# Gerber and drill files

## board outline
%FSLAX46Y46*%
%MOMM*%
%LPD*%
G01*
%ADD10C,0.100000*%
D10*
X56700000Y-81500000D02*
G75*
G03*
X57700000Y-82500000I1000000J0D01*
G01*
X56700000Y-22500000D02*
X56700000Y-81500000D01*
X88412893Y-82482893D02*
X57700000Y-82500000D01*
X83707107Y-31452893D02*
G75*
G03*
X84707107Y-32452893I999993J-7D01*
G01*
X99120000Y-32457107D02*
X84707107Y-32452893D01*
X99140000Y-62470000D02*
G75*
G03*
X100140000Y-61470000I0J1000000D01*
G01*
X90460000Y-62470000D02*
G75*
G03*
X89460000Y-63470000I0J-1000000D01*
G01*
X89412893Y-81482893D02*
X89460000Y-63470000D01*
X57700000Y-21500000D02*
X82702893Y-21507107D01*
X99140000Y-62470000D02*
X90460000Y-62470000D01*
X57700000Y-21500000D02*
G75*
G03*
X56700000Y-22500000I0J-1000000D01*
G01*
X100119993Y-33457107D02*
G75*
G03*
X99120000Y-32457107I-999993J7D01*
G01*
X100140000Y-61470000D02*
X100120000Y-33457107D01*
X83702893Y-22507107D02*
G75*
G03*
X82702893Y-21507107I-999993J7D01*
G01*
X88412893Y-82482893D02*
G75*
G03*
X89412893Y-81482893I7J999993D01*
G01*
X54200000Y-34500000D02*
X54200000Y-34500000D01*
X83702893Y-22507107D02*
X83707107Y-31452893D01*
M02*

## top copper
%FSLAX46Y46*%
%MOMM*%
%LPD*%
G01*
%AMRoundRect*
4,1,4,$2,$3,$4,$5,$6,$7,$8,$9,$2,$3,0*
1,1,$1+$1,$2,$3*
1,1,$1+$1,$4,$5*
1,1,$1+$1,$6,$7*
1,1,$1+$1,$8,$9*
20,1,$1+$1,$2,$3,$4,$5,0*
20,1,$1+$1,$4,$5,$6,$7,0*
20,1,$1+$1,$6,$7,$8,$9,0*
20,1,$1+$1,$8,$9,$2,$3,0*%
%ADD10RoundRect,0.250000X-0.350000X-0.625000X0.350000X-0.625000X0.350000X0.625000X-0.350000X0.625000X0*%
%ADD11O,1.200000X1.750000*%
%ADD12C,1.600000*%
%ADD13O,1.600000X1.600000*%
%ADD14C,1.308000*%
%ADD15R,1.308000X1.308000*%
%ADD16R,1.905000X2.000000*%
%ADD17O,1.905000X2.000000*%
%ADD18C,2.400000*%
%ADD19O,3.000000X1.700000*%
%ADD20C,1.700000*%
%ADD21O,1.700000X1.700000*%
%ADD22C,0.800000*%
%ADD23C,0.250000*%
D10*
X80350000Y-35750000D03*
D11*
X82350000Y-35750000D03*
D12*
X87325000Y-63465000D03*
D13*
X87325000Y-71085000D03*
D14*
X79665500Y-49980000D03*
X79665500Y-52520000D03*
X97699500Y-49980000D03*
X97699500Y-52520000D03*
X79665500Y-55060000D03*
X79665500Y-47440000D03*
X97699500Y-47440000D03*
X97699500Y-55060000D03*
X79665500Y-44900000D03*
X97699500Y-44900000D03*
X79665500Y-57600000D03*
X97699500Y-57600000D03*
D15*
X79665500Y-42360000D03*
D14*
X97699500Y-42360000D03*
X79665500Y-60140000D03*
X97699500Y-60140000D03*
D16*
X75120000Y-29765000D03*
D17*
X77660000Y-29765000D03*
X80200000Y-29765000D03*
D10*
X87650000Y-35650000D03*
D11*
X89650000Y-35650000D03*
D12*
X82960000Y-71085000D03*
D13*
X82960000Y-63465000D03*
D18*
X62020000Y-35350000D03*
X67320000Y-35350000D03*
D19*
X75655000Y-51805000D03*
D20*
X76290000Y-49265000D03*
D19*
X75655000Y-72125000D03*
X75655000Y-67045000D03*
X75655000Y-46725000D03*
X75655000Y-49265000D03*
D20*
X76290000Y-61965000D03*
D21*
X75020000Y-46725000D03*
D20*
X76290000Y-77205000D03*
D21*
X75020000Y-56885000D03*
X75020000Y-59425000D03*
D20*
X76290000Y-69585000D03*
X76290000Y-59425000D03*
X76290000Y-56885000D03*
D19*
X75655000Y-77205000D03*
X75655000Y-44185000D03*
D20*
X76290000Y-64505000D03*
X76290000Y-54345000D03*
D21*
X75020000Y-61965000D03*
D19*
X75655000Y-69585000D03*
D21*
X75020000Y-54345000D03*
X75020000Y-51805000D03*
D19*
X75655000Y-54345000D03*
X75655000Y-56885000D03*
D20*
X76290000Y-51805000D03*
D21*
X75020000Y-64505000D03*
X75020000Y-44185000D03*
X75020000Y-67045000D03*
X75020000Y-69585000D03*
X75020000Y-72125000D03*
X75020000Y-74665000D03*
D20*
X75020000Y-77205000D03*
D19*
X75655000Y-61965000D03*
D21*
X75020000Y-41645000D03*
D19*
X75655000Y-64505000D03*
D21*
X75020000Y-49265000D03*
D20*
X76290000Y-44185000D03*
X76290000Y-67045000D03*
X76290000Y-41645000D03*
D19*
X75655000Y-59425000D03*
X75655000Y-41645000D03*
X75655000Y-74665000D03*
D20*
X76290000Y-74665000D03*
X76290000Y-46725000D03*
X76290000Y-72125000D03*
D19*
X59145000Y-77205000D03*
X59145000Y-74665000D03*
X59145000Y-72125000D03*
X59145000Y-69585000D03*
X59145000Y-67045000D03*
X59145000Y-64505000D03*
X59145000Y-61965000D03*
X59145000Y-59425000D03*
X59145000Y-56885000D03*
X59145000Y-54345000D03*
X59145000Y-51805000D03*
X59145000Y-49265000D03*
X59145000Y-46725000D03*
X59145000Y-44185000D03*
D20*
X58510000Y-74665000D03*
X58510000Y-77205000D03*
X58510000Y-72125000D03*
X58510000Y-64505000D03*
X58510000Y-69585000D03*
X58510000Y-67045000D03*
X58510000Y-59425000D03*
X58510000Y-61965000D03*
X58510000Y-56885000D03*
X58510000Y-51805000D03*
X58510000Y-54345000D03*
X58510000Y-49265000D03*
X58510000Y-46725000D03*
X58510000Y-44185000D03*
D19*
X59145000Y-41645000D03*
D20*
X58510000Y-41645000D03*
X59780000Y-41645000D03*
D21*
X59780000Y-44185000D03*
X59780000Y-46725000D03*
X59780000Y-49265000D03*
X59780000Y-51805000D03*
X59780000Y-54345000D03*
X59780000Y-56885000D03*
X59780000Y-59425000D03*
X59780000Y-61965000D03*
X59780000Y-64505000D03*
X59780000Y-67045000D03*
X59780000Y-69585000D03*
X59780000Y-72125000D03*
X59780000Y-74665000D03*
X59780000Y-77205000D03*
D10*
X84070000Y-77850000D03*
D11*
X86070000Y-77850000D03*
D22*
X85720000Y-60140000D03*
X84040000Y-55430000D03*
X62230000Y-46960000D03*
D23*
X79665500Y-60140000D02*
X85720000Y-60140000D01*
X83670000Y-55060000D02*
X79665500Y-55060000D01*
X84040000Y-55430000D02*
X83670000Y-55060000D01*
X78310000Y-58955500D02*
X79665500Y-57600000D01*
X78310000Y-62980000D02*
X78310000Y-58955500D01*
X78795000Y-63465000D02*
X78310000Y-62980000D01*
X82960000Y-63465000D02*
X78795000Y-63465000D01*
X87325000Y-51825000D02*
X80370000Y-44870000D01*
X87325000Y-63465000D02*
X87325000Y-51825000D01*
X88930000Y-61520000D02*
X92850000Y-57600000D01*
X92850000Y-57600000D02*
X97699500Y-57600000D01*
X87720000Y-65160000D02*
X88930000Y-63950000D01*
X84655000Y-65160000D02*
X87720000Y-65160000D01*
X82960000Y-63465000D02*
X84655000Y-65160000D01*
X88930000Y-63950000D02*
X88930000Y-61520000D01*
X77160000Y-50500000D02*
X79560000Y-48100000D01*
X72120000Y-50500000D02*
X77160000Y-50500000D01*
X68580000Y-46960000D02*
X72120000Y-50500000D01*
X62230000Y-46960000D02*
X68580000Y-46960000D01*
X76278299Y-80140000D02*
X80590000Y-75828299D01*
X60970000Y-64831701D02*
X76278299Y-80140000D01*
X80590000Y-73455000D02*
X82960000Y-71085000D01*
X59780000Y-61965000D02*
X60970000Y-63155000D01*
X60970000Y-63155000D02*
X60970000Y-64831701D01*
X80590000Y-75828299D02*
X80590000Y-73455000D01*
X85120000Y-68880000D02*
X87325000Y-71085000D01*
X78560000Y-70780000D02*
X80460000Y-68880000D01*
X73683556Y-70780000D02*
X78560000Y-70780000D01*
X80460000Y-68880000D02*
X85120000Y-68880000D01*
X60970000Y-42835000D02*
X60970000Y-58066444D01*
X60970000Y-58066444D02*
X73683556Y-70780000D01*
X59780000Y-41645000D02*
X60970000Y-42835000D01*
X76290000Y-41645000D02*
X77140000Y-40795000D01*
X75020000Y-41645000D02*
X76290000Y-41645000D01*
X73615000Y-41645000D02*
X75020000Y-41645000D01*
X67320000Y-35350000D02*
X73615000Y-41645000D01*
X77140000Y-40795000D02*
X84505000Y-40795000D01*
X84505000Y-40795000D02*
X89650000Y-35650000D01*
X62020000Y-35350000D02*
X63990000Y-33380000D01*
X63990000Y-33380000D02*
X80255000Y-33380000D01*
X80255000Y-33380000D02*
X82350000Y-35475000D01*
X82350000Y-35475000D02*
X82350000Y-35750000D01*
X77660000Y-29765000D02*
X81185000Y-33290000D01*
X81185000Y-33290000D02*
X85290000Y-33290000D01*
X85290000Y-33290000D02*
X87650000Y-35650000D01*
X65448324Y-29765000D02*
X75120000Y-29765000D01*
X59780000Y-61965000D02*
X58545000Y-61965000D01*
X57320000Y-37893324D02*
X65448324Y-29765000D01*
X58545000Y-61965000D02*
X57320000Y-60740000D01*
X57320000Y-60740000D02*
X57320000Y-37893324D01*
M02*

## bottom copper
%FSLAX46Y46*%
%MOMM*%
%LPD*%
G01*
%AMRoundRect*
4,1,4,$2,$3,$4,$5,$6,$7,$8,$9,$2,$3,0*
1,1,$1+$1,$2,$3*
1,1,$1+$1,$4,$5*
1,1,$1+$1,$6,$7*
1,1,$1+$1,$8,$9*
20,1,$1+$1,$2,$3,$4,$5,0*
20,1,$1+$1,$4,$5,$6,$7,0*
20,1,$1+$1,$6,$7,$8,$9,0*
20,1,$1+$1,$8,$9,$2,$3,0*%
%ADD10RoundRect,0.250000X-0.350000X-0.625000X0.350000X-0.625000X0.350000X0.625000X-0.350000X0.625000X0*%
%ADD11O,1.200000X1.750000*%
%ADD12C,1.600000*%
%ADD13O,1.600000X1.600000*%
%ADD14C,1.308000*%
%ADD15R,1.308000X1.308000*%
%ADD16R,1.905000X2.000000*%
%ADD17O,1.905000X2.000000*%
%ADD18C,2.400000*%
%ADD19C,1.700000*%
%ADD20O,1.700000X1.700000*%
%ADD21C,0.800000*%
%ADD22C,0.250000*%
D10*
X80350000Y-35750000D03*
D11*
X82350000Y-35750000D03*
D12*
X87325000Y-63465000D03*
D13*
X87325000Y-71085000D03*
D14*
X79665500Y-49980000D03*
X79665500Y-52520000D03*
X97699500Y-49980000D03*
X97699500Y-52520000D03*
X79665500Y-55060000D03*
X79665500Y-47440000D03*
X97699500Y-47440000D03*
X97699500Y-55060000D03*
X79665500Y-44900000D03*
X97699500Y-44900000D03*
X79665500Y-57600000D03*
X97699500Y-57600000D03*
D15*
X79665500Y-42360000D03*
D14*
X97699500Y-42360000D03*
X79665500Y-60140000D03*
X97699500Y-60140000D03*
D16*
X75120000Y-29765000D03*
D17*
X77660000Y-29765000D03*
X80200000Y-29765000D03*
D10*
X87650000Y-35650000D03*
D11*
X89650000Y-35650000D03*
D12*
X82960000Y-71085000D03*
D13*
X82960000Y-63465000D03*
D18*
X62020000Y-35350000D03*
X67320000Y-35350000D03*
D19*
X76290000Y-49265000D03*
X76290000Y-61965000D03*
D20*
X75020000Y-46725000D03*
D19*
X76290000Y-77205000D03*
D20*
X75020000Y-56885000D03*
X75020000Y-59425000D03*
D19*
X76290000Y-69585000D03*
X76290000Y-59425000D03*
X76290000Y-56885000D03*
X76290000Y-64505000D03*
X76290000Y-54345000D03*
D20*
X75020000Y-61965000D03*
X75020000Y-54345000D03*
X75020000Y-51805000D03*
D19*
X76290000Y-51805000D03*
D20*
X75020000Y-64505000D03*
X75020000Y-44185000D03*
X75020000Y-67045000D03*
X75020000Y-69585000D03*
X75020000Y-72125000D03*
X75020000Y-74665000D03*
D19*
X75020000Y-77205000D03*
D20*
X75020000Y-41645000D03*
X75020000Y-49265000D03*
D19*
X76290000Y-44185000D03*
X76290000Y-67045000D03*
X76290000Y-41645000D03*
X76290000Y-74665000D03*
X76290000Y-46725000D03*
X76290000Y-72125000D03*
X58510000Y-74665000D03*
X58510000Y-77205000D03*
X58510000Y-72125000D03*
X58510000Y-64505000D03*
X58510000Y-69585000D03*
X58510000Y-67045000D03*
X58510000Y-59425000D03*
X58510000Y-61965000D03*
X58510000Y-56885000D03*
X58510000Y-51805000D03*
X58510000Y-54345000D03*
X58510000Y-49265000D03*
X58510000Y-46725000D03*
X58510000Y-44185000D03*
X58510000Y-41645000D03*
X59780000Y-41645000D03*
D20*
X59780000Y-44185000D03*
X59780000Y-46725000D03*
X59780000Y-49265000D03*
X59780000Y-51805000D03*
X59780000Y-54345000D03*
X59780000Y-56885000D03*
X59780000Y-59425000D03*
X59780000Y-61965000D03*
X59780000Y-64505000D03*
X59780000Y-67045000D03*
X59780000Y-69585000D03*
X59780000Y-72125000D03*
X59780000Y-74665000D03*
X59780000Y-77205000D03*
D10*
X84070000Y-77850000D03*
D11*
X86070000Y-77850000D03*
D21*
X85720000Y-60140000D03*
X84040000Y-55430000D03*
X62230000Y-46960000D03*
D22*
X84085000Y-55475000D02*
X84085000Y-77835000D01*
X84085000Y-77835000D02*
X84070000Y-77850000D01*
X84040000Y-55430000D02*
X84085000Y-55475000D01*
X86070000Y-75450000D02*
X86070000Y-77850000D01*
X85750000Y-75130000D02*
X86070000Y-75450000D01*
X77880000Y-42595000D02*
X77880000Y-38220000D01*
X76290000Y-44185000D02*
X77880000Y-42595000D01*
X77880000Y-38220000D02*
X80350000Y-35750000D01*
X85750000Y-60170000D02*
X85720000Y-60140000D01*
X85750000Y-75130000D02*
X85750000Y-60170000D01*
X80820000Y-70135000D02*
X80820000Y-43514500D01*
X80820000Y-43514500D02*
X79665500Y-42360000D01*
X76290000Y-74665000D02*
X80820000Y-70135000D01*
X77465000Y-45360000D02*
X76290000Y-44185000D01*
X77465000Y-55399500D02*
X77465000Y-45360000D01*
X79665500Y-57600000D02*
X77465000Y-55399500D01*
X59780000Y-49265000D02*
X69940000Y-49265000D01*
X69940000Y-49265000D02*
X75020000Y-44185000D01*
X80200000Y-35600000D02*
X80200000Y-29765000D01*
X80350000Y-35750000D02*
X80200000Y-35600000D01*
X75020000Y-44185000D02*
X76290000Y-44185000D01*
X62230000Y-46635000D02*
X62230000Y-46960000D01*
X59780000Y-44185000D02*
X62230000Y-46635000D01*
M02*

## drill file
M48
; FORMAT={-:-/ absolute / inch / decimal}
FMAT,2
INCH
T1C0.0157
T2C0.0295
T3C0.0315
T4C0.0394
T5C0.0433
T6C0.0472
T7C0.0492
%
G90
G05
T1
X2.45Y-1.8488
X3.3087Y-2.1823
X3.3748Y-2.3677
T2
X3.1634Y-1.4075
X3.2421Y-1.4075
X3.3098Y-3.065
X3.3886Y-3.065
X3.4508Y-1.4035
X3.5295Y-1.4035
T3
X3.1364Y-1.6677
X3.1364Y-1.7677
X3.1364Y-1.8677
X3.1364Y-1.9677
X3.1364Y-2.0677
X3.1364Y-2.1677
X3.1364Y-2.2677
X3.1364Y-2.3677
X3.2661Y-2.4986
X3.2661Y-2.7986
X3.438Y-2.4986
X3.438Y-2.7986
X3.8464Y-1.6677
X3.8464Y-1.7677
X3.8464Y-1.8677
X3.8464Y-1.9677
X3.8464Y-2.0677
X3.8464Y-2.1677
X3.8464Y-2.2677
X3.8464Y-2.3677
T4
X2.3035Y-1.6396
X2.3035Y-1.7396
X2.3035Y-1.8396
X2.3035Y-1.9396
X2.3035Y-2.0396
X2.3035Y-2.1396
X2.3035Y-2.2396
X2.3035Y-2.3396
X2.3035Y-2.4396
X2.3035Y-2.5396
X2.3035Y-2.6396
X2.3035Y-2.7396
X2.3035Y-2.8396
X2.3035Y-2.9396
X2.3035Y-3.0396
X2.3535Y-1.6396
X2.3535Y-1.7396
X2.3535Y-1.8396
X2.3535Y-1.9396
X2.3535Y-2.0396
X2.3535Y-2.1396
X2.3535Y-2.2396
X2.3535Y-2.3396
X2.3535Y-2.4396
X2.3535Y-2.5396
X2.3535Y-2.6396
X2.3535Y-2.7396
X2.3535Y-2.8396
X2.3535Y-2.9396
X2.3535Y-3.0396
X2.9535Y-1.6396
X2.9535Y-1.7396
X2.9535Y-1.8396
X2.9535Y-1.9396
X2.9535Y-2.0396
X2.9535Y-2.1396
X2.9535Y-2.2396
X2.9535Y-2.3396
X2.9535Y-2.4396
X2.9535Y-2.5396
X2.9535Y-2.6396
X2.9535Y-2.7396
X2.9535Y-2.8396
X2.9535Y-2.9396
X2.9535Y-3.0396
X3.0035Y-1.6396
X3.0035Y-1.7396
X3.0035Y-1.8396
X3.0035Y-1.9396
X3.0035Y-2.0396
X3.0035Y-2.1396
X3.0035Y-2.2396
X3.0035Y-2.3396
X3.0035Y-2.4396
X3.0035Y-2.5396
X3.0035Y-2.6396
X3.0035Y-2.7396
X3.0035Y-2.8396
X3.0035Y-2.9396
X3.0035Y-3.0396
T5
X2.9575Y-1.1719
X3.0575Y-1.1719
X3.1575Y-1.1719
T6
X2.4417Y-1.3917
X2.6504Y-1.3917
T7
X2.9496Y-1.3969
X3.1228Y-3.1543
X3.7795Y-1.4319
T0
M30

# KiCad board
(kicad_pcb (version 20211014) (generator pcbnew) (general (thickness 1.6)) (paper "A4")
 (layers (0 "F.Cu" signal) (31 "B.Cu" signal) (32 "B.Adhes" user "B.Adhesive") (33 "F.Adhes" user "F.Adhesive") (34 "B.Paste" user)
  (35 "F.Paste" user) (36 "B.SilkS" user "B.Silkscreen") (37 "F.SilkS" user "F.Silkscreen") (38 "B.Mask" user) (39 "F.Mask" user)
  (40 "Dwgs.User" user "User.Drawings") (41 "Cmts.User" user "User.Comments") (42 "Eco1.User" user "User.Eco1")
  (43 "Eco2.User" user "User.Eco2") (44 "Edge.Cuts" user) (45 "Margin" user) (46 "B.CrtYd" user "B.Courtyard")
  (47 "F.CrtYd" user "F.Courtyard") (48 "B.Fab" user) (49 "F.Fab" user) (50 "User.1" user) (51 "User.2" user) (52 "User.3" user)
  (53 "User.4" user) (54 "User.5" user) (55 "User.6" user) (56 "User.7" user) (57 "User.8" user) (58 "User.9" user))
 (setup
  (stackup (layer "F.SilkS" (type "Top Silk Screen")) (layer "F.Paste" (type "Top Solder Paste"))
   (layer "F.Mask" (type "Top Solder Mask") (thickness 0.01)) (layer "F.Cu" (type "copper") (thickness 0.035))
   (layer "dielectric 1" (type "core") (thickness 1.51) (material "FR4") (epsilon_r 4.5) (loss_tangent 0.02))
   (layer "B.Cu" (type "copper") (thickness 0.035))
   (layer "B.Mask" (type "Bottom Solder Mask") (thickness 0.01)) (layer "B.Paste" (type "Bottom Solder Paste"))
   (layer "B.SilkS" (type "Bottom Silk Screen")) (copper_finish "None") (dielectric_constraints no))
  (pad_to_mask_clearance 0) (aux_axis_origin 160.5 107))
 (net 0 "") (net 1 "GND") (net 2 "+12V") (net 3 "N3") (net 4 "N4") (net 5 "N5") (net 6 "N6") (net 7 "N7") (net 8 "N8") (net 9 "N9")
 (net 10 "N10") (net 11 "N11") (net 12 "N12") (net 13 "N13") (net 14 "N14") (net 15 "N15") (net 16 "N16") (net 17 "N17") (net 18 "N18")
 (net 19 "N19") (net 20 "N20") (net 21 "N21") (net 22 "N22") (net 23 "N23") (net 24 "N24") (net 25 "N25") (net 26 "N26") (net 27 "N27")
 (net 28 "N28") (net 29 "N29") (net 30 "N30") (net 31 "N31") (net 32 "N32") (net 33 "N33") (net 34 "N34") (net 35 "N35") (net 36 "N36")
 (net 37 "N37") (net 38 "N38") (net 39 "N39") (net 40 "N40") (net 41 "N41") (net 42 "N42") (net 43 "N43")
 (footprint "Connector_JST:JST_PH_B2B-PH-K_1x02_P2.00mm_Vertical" (layer "F.Cu") (at 80.35 35.75)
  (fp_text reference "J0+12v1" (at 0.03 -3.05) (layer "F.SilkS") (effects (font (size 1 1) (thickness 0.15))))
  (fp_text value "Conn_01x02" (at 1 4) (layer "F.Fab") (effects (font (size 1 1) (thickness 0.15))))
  (pad "1" thru_hole roundrect (at 0 0) (size 1.2 1.75) (drill 0.75) (layers *.Cu *.Mask) (roundrect_rratio 0.208333) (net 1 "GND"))
  (pad "2" thru_hole oval (at 2 0) (size 1.2 1.75) (drill 0.75) (layers *.Cu *.Mask) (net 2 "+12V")))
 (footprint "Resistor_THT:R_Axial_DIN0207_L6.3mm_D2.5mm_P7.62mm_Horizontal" (layer "F.Cu") (at 87.325 63.465 -90)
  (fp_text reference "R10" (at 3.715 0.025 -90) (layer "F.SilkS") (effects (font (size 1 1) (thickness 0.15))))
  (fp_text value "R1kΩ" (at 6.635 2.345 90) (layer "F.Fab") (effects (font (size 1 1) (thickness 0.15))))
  (pad "1" thru_hole circle (at 0 0 270) (size 1.6 1.6) (drill 0.8) (layers *.Cu *.Mask) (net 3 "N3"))
  (pad "2" thru_hole oval (at 7.62 0 270) (size 1.6 1.6) (drill 0.8) (layers *.Cu *.Mask) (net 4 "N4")))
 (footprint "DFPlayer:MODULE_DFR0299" (layer "F.Cu") (at 88.6825 51.25)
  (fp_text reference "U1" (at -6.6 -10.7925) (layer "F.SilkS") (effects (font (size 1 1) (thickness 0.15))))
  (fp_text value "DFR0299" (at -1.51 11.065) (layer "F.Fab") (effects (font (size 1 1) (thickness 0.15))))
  (pad "1" thru_hole rect locked (at -9.017 -8.89) (size 1.308 1.308) (drill 0.8) (layers *.Cu *.Mask) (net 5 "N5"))
  (pad "2" thru_hole circle locked (at -9.017 -6.35) (size 1.308 1.308) (drill 0.8) (layers *.Cu *.Mask) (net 3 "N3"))
  (pad "3" thru_hole circle locked (at -9.017 -3.81) (size 1.308 1.308) (drill 0.8) (layers *.Cu *.Mask) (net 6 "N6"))
  (pad "4" thru_hole circle locked (at -9.017 -1.27) (size 1.308 1.308) (drill 0.8) (layers *.Cu *.Mask) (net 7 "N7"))
  (pad "5" thru_hole circle locked (at -9.017 1.27) (size 1.308 1.308) (drill 0.8) (layers *.Cu *.Mask) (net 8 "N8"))
  (pad "6" thru_hole circle locked (at -9.017 3.81) (size 1.308 1.308) (drill 0.8) (layers *.Cu *.Mask) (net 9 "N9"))
  (pad "7" thru_hole circle locked (at -9.017 6.35) (size 1.308 1.308) (drill 0.8) (layers *.Cu *.Mask) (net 1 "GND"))
  (pad "8" thru_hole circle locked (at -9.017 8.89) (size 1.308 1.308) (drill 0.8) (layers *.Cu *.Mask) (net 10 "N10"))
  (pad "9" thru_hole circle locked (at 9.017 8.89) (size 1.308 1.308) (drill 0.8) (layers *.Cu *.Mask) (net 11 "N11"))
  (pad "10" thru_hole circle locked (at 9.017 6.35) (size 1.308 1.308) (drill 0.8) (layers *.Cu *.Mask) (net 1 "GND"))
  (pad "11" thru_hole circle locked (at 9.017 3.81) (size 1.308 1.308) (drill 0.8) (layers *.Cu *.Mask) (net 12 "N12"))
  (pad "12" thru_hole circle locked (at 9.017 1.27) (size 1.308 1.308) (drill 0.8) (layers *.Cu *.Mask) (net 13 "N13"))
  (pad "13" thru_hole circle locked (at 9.017 -1.27) (size 1.308 1.308) (drill 0.8) (layers *.Cu *.Mask) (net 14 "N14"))
  (pad "14" thru_hole circle locked (at 9.017 -3.81) (size 1.308 1.308) (drill 0.8) (layers *.Cu *.Mask) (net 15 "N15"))
  (pad "15" thru_hole circle locked (at 9.017 -6.35) (size 1.308 1.308) (drill 0.8) (layers *.Cu *.Mask) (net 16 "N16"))
  (pad "16" thru_hole circle locked (at 9.017 -8.89) (size 1.308 1.308) (drill 0.8) (layers *.Cu *.Mask) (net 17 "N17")))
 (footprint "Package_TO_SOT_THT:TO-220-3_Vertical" (layer "F.Cu") (at 75.12 29.765)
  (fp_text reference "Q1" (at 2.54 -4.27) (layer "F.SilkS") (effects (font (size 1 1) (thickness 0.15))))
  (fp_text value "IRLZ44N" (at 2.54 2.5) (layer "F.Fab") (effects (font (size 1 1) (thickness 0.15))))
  (pad "1" thru_hole rect (at 0 0) (size 1.905 2) (drill 1.1) (layers *.Cu *.Mask) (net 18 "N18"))
  (pad "2" thru_hole oval (at 2.54 0) (size 1.905 2) (drill 1.1) (layers *.Cu *.Mask) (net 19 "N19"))
  (pad "3" thru_hole oval (at 5.08 0) (size 1.905 2) (drill 1.1) (layers *.Cu *.Mask) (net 1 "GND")))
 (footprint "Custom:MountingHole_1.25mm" (layer "F.Cu") (at 96 36.37)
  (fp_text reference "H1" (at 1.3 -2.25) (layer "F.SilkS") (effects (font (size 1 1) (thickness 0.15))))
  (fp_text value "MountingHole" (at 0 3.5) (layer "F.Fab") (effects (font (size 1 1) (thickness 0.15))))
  (pad "" np_thru_hole circle (at 0 0) (size 1.25 1.25) (drill 1.25) (layers F&B.Cu *.Mask)))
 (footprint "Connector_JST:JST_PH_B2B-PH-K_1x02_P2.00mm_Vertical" (layer "F.Cu") (at 87.65 35.65)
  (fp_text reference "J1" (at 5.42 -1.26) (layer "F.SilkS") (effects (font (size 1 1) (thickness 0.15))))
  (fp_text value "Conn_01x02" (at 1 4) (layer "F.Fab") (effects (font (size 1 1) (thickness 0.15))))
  (pad "1" thru_hole roundrect (at 0 0) (size 1.2 1.75) (drill 0.75) (layers *.Cu *.Mask) (roundrect_rratio 0.208333) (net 19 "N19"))
  (pad "2" thru_hole oval (at 2 0) (size 1.2 1.75) (drill 0.75) (layers *.Cu *.Mask) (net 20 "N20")))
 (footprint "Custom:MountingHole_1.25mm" (layer "F.Cu") (at 79.32 80.12)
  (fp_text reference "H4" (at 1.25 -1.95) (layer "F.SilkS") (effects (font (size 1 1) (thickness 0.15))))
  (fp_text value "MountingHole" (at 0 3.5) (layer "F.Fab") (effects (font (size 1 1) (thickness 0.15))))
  (pad "" np_thru_hole circle (at 0 0) (size 1.25 1.25) (drill 1.25) (layers F&B.Cu *.Mask)))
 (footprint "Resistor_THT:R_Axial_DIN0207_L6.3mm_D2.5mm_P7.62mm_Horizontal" (layer "F.Cu") (at 82.96 71.085 90)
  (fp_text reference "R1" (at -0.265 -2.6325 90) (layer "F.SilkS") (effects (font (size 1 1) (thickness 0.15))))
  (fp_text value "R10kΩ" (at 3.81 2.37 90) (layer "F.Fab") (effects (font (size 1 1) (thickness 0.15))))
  (pad "1" thru_hole circle (at 0 0 90) (size 1.6 1.6) (drill 0.8) (layers *.Cu *.Mask) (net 18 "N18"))
  (pad "2" thru_hole oval (at 7.62 0 90) (size 1.6 1.6) (drill 0.8) (layers *.Cu *.Mask) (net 1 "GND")))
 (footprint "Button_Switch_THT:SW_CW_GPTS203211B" (layer "F.Cu") (at 62.02 35.35 90)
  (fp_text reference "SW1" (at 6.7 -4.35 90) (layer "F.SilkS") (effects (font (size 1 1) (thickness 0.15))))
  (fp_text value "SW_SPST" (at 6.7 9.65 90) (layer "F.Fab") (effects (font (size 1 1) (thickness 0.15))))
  (pad "1" thru_hole circle (at 0 0 90) (size 2.4 2.4) (drill 1.2) (layers *.Cu *.Mask) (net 2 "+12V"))
  (pad "2" thru_hole circle (at 0 5.3 90) (size 2.4 2.4) (drill 1.2) (layers *.Cu *.Mask) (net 20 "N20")))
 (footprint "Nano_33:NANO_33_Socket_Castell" (layer "F.Cu") (at 67.4 59.425 90)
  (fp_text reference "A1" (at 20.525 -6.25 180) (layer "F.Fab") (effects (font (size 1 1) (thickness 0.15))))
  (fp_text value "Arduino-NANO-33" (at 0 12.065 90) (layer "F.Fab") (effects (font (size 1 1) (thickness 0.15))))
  (pad "1" thru_hole circle locked (at -17.78 7.62 180) (size 1.7 1.7) (drill 1) (layers *.Cu *.Mask) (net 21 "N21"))
  (pad "1" smd oval locked (at -17.78 8.255 180) (size 3 1.7) (layers "F.Cu" "F.Mask") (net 21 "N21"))
  (pad "1" thru_hole circle locked (at -17.78 8.89 180) (size 1.7 1.7) (drill 1) (layers *.Cu *.Mask) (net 21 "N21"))
  (pad "2" thru_hole oval locked (at -15.24 7.62 180) (size 1.7 1.7) (drill 1) (layers *.Cu *.Mask) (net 5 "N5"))
  (pad "2" smd oval locked (at -15.24 8.255 180) (size 3 1.7) (layers "F.Cu" "F.Mask") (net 5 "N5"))
  (pad "2" thru_hole circle locked (at -15.24 8.89 180) (size 1.7 1.7) (drill 1) (layers *.Cu *.Mask) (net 5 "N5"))
  (pad "3" smd oval locked (at -12.7 8.255 180) (size 3 1.7) (layers "F.Cu" "F.Mask") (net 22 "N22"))
  (pad "3" thru_hole oval locked (at -12.7 7.62 180) (size 1.7 1.7) (drill 1) (layers *.Cu *.Mask) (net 22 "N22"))
  (pad "3" thru_hole circle locked (at -12.7 8.89 180) (size 1.7 1.7) (drill 1) (layers *.Cu *.Mask) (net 22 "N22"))
  (pad "4" thru_hole circle locked (at -10.16 8.89 180) (size 1.7 1.7) (drill 1) (layers *.Cu *.Mask) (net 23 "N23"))
  (pad "4" smd oval locked (at -10.16 8.255 180) (size 3 1.7) (layers "F.Cu" "F.Mask") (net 23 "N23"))
  (pad "4" thru_hole oval locked (at -10.16 7.62 180) (size 1.7 1.7) (drill 1) (layers *.Cu *.Mask) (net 23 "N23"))
  (pad "5" thru_hole circle locked (at -7.62 8.89 180) (size 1.7 1.7) (drill 1) (layers *.Cu *.Mask) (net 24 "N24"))
  (pad "5" thru_hole oval locked (at -7.62 7.62 180) (size 1.7 1.7) (drill 1) (layers *.Cu *.Mask) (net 24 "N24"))
  (pad "5" smd oval locked (at -7.62 8.255 180) (size 3 1.7) (layers "F.Cu" "F.Mask") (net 24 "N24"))
  (pad "6" smd oval locked (at -5.08 8.255 180) (size 3 1.7) (layers "F.Cu" "F.Mask") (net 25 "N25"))
  (pad "6" thru_hole circle locked (at -5.08 8.89 180) (size 1.7 1.7) (drill 1) (layers *.Cu *.Mask) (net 25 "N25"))
  (pad "6" thru_hole oval locked (at -5.08 7.62 180) (size 1.7 1.7) (drill 1) (layers *.Cu *.Mask) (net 25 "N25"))
  (pad "7" thru_hole circle locked (at -2.54 8.89 180) (size 1.7 1.7) (drill 1) (layers *.Cu *.Mask) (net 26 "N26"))
  (pad "7" thru_hole oval locked (at -2.54 7.62 180) (size 1.7 1.7) (drill 1) (layers *.Cu *.Mask) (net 26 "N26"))
  (pad "7" smd oval locked (at -2.54 8.255 180) (size 3 1.7) (layers "F.Cu" "F.Mask") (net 26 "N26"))
  (pad "8" thru_hole oval locked (at 0 7.62 180) (size 1.7 1.7) (drill 1) (layers *.Cu *.Mask) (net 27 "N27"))
  (pad "8" smd oval locked (at 0 8.255 180) (size 3 1.7) (layers "F.Cu" "F.Mask") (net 27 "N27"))
  (pad "8" thru_hole circle locked (at 0 8.89 180) (size 1.7 1.7) (drill 1) (layers *.Cu *.Mask) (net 27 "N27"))
  (pad "9" thru_hole circle locked (at 2.54 8.89 180) (size 1.7 1.7) (drill 1) (layers *.Cu *.Mask) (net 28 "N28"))
  (pad "9" thru_hole oval locked (at 2.54 7.62 180) (size 1.7 1.7) (drill 1) (layers *.Cu *.Mask) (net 28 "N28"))
  (pad "9" smd oval locked (at 2.54 8.255 180) (size 3 1.7) (layers "F.Cu" "F.Mask") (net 28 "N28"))
  (pad "10" thru_hole oval locked (at 5.08 7.62 180) (size 1.7 1.7) (drill 1) (layers *.Cu *.Mask) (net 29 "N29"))
  (pad "10" smd oval locked (at 5.08 8.255 180) (size 3 1.7) (layers "F.Cu" "F.Mask") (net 29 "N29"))
  (pad "10" thru_hole circle locked (at 5.08 8.89 180) (size 1.7 1.7) (drill 1) (layers *.Cu *.Mask) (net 29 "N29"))
  (pad "11" thru_hole oval locked (at 7.62 7.62 180) (size 1.7 1.7) (drill 1) (layers *.Cu *.Mask) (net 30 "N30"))
  (pad "11" smd oval locked (at 7.62 8.255 180) (size 3 1.7) (layers "F.Cu" "F.Mask") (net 30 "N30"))
  (pad "11" thru_hole circle locked (at 7.62 8.89 180) (size 1.7 1.7) (drill 1) (layers *.Cu *.Mask) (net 30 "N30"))
  (pad "12" thru_hole circle locked (at 10.16 8.89 180) (size 1.7 1.7) (drill 1) (layers *.Cu *.Mask) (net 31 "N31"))
  (pad "12" thru_hole oval locked (at 10.16 7.62 180) (size 1.7 1.7) (drill 1) (layers *.Cu *.Mask) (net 31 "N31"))
  (pad "12" smd oval locked (at 10.16 8.255 180) (size 3 1.7) (layers "F.Cu" "F.Mask") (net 31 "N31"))
  (pad "13" thru_hole circle locked (at 12.7 8.89 180) (size 1.7 1.7) (drill 1) (layers *.Cu *.Mask) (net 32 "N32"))
  (pad "13" smd oval locked (at 12.7 8.255 180) (size 3 1.7) (layers "F.Cu" "F.Mask") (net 32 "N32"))
  (pad "13" thru_hole oval locked (at 12.7 7.62 180) (size 1.7 1.7) (drill 1) (layers *.Cu *.Mask) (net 32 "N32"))
  (pad "14" thru_hole circle locked (at 15.24 8.89 180) (size 1.7 1.7) (drill 1) (layers *.Cu *.Mask) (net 1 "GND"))
  (pad "14" thru_hole oval locked (at 15.24 7.62 180) (size 1.7 1.7) (drill 1) (layers *.Cu *.Mask) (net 1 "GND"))
  (pad "14" smd oval locked (at 15.24 8.255 180) (size 3 1.7) (layers "F.Cu" "F.Mask") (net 1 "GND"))
  (pad "15" smd oval locked (at 17.78 8.255 180) (size 3 1.7) (layers "F.Cu" "F.Mask") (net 20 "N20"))
  (pad "15" thru_hole circle locked (at 17.78 8.89 180) (size 1.7 1.7) (drill 1) (layers *.Cu *.Mask) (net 20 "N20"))
  (pad "15" thru_hole oval locked (at 17.78 7.62 180) (size 1.7 1.7) (drill 1) (layers *.Cu *.Mask) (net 20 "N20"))
  (pad "16" thru_hole circle locked (at 17.78 -8.89) (size 1.7 1.7) (drill 1) (layers *.Cu *.Mask) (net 4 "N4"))
  (pad "16" thru_hole circle locked (at 17.78 -7.62) (size 1.7 1.7) (drill 1) (layers *.Cu *.Mask) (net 4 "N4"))
  (pad "16" smd oval locked (at 17.78 -8.255) (size 3 1.7) (layers "F.Cu" "F.Mask") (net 4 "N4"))
  (pad "17" thru_hole oval locked (at 15.24 -7.62) (size 1.7 1.7) (drill 1) (layers *.Cu *.Mask) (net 6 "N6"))
  (pad "17" thru_hole circle locked (at 15.24 -8.89) (size 1.7 1.7) (drill 1) (layers *.Cu *.Mask) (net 6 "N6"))
  (pad "17" smd oval locked (at 15.24 -8.255) (size 3 1.7) (layers "F.Cu" "F.Mask") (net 6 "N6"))
  (pad "18" thru_hole oval locked (at 12.7 -7.62) (size 1.7 1.7) (drill 1) (layers *.Cu *.Mask) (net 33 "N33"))
  (pad "18" thru_hole circle locked (at 12.7 -8.89) (size 1.7 1.7) (drill 1) (layers *.Cu *.Mask) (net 33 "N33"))
  (pad "18" smd oval locked (at 12.7 -8.255) (size 3 1.7) (layers "F.Cu" "F.Mask") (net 33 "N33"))
  (pad "19" thru_hole oval locked (at 10.16 -7.62) (size 1.7 1.7) (drill 1) (layers *.Cu *.Mask) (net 1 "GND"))
  (pad "19" thru_hole circle locked (at 10.16 -8.89) (size 1.7 1.7) (drill 1) (layers *.Cu *.Mask) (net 1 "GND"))
  (pad "19" smd oval locked (at 10.16 -8.255) (size 3 1.7) (layers "F.Cu" "F.Mask") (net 1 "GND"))
  (pad "20" thru_hole circle locked (at 7.62 -8.89) (size 1.7 1.7) (drill 1) (layers *.Cu *.Mask) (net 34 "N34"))
  (pad "20" thru_hole oval locked (at 7.62 -7.62) (size 1.7 1.7) (drill 1) (layers *.Cu *.Mask) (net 34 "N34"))
  (pad "20" smd oval locked (at 7.62 -8.255) (size 3 1.7) (layers "F.Cu" "F.Mask") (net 34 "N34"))
  (pad "21" thru_hole circle locked (at 5.08 -8.89) (size 1.7 1.7) (drill 1) (layers *.Cu *.Mask) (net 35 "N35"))
  (pad "21" thru_hole oval locked (at 5.08 -7.62) (size 1.7 1.7) (drill 1) (layers *.Cu *.Mask) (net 35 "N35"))
  (pad "21" smd oval locked (at 5.08 -8.255) (size 3 1.7) (layers "F.Cu" "F.Mask") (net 35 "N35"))
  (pad "22" thru_hole circle locked (at 2.54 -8.89) (size 1.7 1.7) (drill 1) (layers *.Cu *.Mask) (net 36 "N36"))
  (pad "22" thru_hole oval locked (at 2.54 -7.62) (size 1.7 1.7) (drill 1) (layers *.Cu *.Mask) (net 36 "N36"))
  (pad "22" smd oval locked (at 2.54 -8.255) (size 3 1.7) (layers "F.Cu" "F.Mask") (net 36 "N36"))
  (pad "23" thru_hole circle locked (at 0 -8.89) (size 1.7 1.7) (drill 1) (layers *.Cu *.Mask) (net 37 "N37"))
  (pad "23" smd oval locked (at 0 -8.255) (size 3 1.7) (layers "F.Cu" "F.Mask") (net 37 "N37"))
  (pad "23" thru_hole oval locked (at 0 -7.62) (size 1.7 1.7) (drill 1) (layers *.Cu *.Mask) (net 37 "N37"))
  (pad "24" thru_hole oval locked (at -2.54 -7.62) (size 1.7 1.7) (drill 1) (layers *.Cu *.Mask) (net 18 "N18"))
  (pad "24" thru_hole circle locked (at -2.54 -8.89) (size 1.7 1.7) (drill 1) (layers *.Cu *.Mask) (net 18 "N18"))
  (pad "24" smd oval locked (at -2.54 -8.255) (size 3 1.7) (layers "F.Cu" "F.Mask") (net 18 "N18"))
  (pad "25" thru_hole oval locked (at -5.08 -7.62) (size 1.7 1.7) (drill 1) (layers *.Cu *.Mask) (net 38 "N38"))
  (pad "25" smd oval locked (at -5.08 -8.255) (size 3 1.7) (layers "F.Cu" "F.Mask") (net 38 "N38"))
  (pad "25" thru_hole circle locked (at -5.08 -8.89) (size 1.7 1.7) (drill 1) (layers *.Cu *.Mask) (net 38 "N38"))
  (pad "26" thru_hole circle locked (at -7.62 -8.89) (size 1.7 1.7) (drill 1) (layers *.Cu *.Mask) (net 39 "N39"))
  (pad "26" thru_hole oval locked (at -7.62 -7.62) (size 1.7 1.7) (drill 1) (layers *.Cu *.Mask) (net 39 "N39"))
  (pad "26" smd oval locked (at -7.62 -8.255) (size 3 1.7) (layers "F.Cu" "F.Mask") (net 39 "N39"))
  (pad "27" thru_hole circle locked (at -10.16 -8.89) (size 1.7 1.7) (drill 1) (layers *.Cu *.Mask) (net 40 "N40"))
  (pad "27" thru_hole oval locked (at -10.16 -7.62) (size 1.7 1.7) (drill 1) (layers *.Cu *.Mask) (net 40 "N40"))
  (pad "27" smd oval locked (at -10.16 -8.255) (size 3 1.7) (layers "F.Cu" "F.Mask") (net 40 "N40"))
  (pad "28" thru_hole circle locked (at -12.7 -8.89) (size 1.7 1.7) (drill 1) (layers *.Cu *.Mask) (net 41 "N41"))
  (pad "28" thru_hole oval locked (at -12.7 -7.62) (size 1.7 1.7) (drill 1) (layers *.Cu *.Mask) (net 41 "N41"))
  (pad "28" smd oval locked (at -12.7 -8.255) (size 3 1.7) (layers "F.Cu" "F.Mask") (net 41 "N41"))
  (pad "29" thru_hole oval locked (at -15.24 -7.62) (size 1.7 1.7) (drill 1) (layers *.Cu *.Mask) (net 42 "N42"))
  (pad "29" thru_hole circle locked (at -15.24 -8.89) (size 1.7 1.7) (drill 1) (layers *.Cu *.Mask) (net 42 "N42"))
  (pad "29" smd oval locked (at -15.24 -8.255) (size 3 1.7) (layers "F.Cu" "F.Mask") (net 42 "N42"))
  (pad "30" smd oval locked (at -17.78 -8.255) (size 3 1.7) (layers "F.Cu" "F.Mask") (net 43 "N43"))
  (pad "30" thru_hole oval locked (at -17.78 -7.62) (size 1.7 1.7) (drill 1) (layers *.Cu *.Mask) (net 43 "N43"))
  (pad "30" thru_hole circle locked (at -17.78 -8.89) (size 1.7 1.7) (drill 1) (layers *.Cu *.Mask) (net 43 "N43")))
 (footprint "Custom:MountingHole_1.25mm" (layer "F.Cu") (at 74.92 35.48)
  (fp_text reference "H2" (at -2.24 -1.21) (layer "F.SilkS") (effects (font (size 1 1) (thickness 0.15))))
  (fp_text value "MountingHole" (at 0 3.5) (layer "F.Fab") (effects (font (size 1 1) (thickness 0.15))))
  (pad "" np_thru_hole circle (at 0 0) (size 1.25 1.25) (drill 1.25) (layers F&B.Cu *.Mask)))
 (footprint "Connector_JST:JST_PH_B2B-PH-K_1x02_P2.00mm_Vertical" (layer "F.Cu") (at 84.07 77.85)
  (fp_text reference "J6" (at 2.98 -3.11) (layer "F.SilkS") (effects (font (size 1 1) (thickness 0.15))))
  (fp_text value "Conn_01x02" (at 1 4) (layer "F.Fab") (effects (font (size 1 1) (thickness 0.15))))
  (pad "1" thru_hole roundrect (at 0 0) (size 1.2 1.75) (drill 0.75) (layers *.Cu *.Mask) (roundrect_rratio 0.208333) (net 9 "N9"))
  (pad "2" thru_hole oval (at 2 0) (size 1.2 1.75) (drill 0.75) (layers *.Cu *.Mask) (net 10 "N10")))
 (gr_arc (start 57.7 82.5) (mid 56.992893 82.207107) (end 56.7 81.5) (layer "Edge.Cuts") (width 0.1))
 (gr_line (start 56.7 22.5) (end 56.7 81.5) (layer "Edge.Cuts") (width 0.1))
 (gr_line (start 88.412893 82.482893) (end 57.7 82.5) (layer "Edge.Cuts") (width 0.1))
 (gr_arc (start 84.707107 32.452893) (mid 84 32.16) (end 83.707107 31.452893) (layer "Edge.Cuts") (width 0.1))
 (gr_line (start 99.12 32.457107) (end 84.707107 32.452893) (layer "Edge.Cuts") (width 0.1))
 (gr_arc (start 100.14 61.47) (mid 99.847107 62.177107) (end 99.14 62.47) (layer "Edge.Cuts") (width 0.1))
 (gr_arc (start 89.46 63.47) (mid 89.752893 62.762893) (end 90.46 62.47) (layer "Edge.Cuts") (width 0.1))
 (gr_line (start 89.412893 81.482893) (end 89.46 63.47) (layer "Edge.Cuts") (width 0.1))
 (gr_line (start 57.7 21.5) (end 82.702893 21.507107) (layer "Edge.Cuts") (width 0.1))
 (gr_line (start 99.14 62.47) (end 90.46 62.47) (layer "Edge.Cuts") (width 0.1))
 (gr_arc (start 56.7 22.5) (mid 56.992893 21.792893) (end 57.7 21.5) (layer "Edge.Cuts") (width 0.1))
 (gr_arc (start 99.12 32.457107) (mid 99.827107 32.75) (end 100.12 33.457107) (layer "Edge.Cuts") (width 0.1))
 (gr_line (start 100.14 61.47) (end 100.12 33.457107) (layer "Edge.Cuts") (width 0.1))
 (gr_arc (start 82.702893 21.507107) (mid 83.41 21.8) (end 83.702893 22.507107) (layer "Edge.Cuts") (width 0.1))
 (gr_arc (start 89.412893 81.482893) (mid 89.12 82.19) (end 88.412893 82.482893) (layer "Edge.Cuts") (width 0.1))
 (gr_line (start 54.2 34.5) (end 54.2 34.5) (layer "Edge.Cuts") (width 0.1))
 (gr_line (start 83.702893 22.507107) (end 83.707107 31.452893) (layer "Edge.Cuts") (width 0.1))
 (segment (start 80.82 70.135) (end 80.82 43.5145) (width 0.25) (layer "B.Cu") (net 5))
 (segment (start 80.82 43.5145) (end 79.6655 42.36) (width 0.25) (layer "B.Cu") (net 5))
 (segment (start 76.29 74.665) (end 80.82 70.135) (width 0.25) (layer "B.Cu") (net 5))
 (segment (start 60.97 42.835) (end 60.97 58.066444) (width 0.25) (layer "F.Cu") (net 4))
 (segment (start 60.97 58.066444) (end 73.683556 70.78) (width 0.25) (layer "F.Cu") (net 4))
 (segment (start 73.683556 70.78) (end 78.56 70.78) (width 0.25) (layer "F.Cu") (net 4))
 (segment (start 85.12 68.88) (end 87.325 71.085) (width 0.25) (layer "F.Cu") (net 4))
 (segment (start 59.78 41.645) (end 60.97 42.835) (width 0.25) (layer "F.Cu") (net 4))
 (segment (start 78.56 70.78) (end 80.46 68.88) (width 0.25) (layer "F.Cu") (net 4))
 (segment (start 80.46 68.88) (end 85.12 68.88) (width 0.25) (layer "F.Cu") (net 4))
 (segment (start 76.29 41.645) (end 77.14 40.795) (width 0.25) (layer "F.Cu") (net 20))
 (segment (start 75.02 41.645) (end 76.29 41.645) (width 0.25) (layer "F.Cu") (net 20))
 (segment (start 73.615 41.645) (end 75.02 41.645) (width 0.25) (layer "F.Cu") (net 20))
 (segment (start 67.32 35.35) (end 73.615 41.645) (width 0.25) (layer "F.Cu") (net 20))
 (segment (start 77.14 40.795) (end 84.505 40.795) (width 0.25) (layer "F.Cu") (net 20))
 (segment (start 84.505 40.795) (end 89.65 35.65) (width 0.25) (layer "F.Cu") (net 20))
 (segment (start 78.31 58.9555) (end 79.6655 57.6) (width 0.25) (layer "F.Cu") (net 1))
 (segment (start 87.72 65.16) (end 88.93 63.95) (width 0.25) (layer "F.Cu") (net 1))
 (segment (start 78.795 63.465) (end 78.31 62.98) (width 0.25) (layer "F.Cu") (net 1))
 (segment (start 88.93 63.95) (end 88.93 61.52) (width 0.25) (layer "F.Cu") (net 1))
 (segment (start 82.96 63.465) (end 84.655 65.16) (width 0.25) (layer "F.Cu") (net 1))
 (segment (start 88.93 61.52) (end 92.85 57.6) (width 0.25) (layer "F.Cu") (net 1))
 (segment (start 84.655 65.16) (end 87.72 65.16) (width 0.25) (layer "F.Cu") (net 1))
 (segment (start 78.31 62.98) (end 78.31 58.9555) (width 0.25) (layer "F.Cu") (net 1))
 (segment (start 92.85 57.6) (end 97.6995 57.6) (width 0.25) (layer "F.Cu") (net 1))
 (segment (start 82.96 63.465) (end 78.795 63.465) (width 0.25) (layer "F.Cu") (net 1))
 (segment (start 77.465 55.3995) (end 77.465 45.36) (width 0.25) (layer "B.Cu") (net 1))
 (segment (start 59.78 49.265) (end 69.94 49.265) (width 0.25) (layer "B.Cu") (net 1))
 (segment (start 69.94 49.265) (end 75.02 44.185) (width 0.25) (layer "B.Cu") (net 1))
 (segment (start 77.465 45.36) (end 76.29 44.185) (width 0.25) (layer "B.Cu") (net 1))
 (segment (start 80.2 35.6) (end 80.2 29.765) (width 0.25) (layer "B.Cu") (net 1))
 (segment (start 80.35 35.75) (end 80.2 35.6) (width 0.25) (layer "B.Cu") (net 1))
 (segment (start 79.6655 57.6) (end 77.465 55.3995) (width 0.25) (layer "B.Cu") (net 1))
 (segment (start 76.29 44.185) (end 77.88 42.595) (width 0.25) (layer "B.Cu") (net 1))
 (segment (start 75.02 44.185) (end 76.29 44.185) (width 0.25) (layer "B.Cu") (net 1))
 (segment (start 77.88 42.595) (end 77.88 38.22) (width 0.25) (layer "B.Cu") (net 1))
 (segment (start 77.88 38.22) (end 80.35 35.75) (width 0.25) (layer "B.Cu") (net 1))
 (segment (start 62.02 35.35) (end 63.99 33.38) (width 0.25) (layer "F.Cu") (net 2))
 (segment (start 63.99 33.38) (end 80.255 33.38) (width 0.25) (layer "F.Cu") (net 2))
 (segment (start 80.255 33.38) (end 82.35 35.475) (width 0.25) (layer "F.Cu") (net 2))
 (segment (start 82.35 35.475) (end 82.35 35.75) (width 0.25) (layer "F.Cu") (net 2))
 (segment (start 77.66 29.765) (end 81.185 33.29) (width 0.25) (layer "F.Cu") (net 19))
 (segment (start 81.185 33.29) (end 85.29 33.29) (width 0.25) (layer "F.Cu") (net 19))
 (segment (start 85.29 33.29) (end 87.65 35.65) (width 0.25) (layer "F.Cu") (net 19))
 (segment (start 59.78 61.965) (end 60.97 63.155) (width 0.25) (layer "F.Cu") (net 18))
 (segment (start 65.448324 29.765) (end 75.12 29.765) (width 0.25) (layer "F.Cu") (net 18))
 (segment (start 59.78 61.965) (end 58.545 61.965) (width 0.25) (layer "F.Cu") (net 18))
 (segment (start 80.59 75.828299) (end 80.59 73.455) (width 0.25) (layer "F.Cu") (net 18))
 (segment (start 57.32 37.893324) (end 65.448324 29.765) (width 0.25) (layer "F.Cu") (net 18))
 (segment (start 58.545 61.965) (end 57.32 60.74) (width 0.25) (layer "F.Cu") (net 18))
 (segment (start 60.97 63.155) (end 60.97 64.831701) (width 0.25) (layer "F.Cu") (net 18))
 (segment (start 80.59 73.455) (end 82.96 71.085) (width 0.25) (layer "F.Cu") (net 18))
 (segment (start 76.278299 80.14) (end 80.59 75.828299) (width 0.25) (layer "F.Cu") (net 18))
 (segment (start 60.97 64.831701) (end 76.278299 80.14) (width 0.25) (layer "F.Cu") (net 18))
 (segment (start 57.32 60.74) (end 57.32 37.893324) (width 0.25) (layer "F.Cu") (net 18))
 (segment (start 77.16 50.5) (end 79.56 48.1) (width 0.25) (layer "F.Cu") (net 6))
 (segment (start 62.23 46.96) (end 68.58 46.96) (width 0.25) (layer "F.Cu") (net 6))
 (segment (start 68.58 46.96) (end 72.12 50.5) (width 0.25) (layer "F.Cu") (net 6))
 (segment (start 72.12 50.5) (end 77.16 50.5) (width 0.25) (layer "F.Cu") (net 6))
 (via (at 62.23 46.96) (size 0.8) (drill 0.4) (layers "F.Cu" "B.Cu") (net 6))
 (segment (start 62.23 46.635) (end 62.23 46.96) (width 0.25) (layer "B.Cu") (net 6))
 (segment (start 59.78 44.185) (end 62.23 46.635) (width 0.25) (layer "B.Cu") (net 6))
 (segment (start 87.325 63.465) (end 87.325 51.825) (width 0.25) (layer "F.Cu") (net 3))
 (segment (start 87.325 51.825) (end 80.37 44.87) (width 0.25) (layer "F.Cu") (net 3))
 (segment (start 83.67 55.06) (end 79.6655 55.06) (width 0.25) (layer "F.Cu") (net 9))
 (segment (start 84.04 55.43) (end 83.67 55.06) (width 0.25) (layer "F.Cu") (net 9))
 (via (at 84.04 55.43) (size 0.8) (drill 0.4) (layers "F.Cu" "B.Cu") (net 9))
 (segment (start 84.04 55.43) (end 84.085 55.475) (width 0.25) (layer "B.Cu") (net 9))
 (segment (start 84.085 55.475) (end 84.085 77.835) (width 0.25) (layer "B.Cu") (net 9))
 (segment (start 84.085 77.835) (end 84.07 77.85) (width 0.25) (layer "B.Cu") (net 9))
 (segment (start 79.6655 60.14) (end 85.72 60.14) (width 0.25) (layer "F.Cu") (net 10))
 (via (at 85.72 60.14) (size 0.8) (drill 0.4) (layers "F.Cu" "B.Cu") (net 10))
 (segment (start 85.75 75.13) (end 85.75 60.17) (width 0.25) (layer "B.Cu") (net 10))
 (segment (start 86.07 75.45) (end 86.07 77.85) (width 0.25) (layer "B.Cu") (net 10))
 (segment (start 85.75 60.17) (end 85.72 60.14) (width 0.25) (layer "B.Cu") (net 10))
 (segment (start 85.75 75.13) (end 86.07 75.45) (width 0.25) (layer "B.Cu") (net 10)))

